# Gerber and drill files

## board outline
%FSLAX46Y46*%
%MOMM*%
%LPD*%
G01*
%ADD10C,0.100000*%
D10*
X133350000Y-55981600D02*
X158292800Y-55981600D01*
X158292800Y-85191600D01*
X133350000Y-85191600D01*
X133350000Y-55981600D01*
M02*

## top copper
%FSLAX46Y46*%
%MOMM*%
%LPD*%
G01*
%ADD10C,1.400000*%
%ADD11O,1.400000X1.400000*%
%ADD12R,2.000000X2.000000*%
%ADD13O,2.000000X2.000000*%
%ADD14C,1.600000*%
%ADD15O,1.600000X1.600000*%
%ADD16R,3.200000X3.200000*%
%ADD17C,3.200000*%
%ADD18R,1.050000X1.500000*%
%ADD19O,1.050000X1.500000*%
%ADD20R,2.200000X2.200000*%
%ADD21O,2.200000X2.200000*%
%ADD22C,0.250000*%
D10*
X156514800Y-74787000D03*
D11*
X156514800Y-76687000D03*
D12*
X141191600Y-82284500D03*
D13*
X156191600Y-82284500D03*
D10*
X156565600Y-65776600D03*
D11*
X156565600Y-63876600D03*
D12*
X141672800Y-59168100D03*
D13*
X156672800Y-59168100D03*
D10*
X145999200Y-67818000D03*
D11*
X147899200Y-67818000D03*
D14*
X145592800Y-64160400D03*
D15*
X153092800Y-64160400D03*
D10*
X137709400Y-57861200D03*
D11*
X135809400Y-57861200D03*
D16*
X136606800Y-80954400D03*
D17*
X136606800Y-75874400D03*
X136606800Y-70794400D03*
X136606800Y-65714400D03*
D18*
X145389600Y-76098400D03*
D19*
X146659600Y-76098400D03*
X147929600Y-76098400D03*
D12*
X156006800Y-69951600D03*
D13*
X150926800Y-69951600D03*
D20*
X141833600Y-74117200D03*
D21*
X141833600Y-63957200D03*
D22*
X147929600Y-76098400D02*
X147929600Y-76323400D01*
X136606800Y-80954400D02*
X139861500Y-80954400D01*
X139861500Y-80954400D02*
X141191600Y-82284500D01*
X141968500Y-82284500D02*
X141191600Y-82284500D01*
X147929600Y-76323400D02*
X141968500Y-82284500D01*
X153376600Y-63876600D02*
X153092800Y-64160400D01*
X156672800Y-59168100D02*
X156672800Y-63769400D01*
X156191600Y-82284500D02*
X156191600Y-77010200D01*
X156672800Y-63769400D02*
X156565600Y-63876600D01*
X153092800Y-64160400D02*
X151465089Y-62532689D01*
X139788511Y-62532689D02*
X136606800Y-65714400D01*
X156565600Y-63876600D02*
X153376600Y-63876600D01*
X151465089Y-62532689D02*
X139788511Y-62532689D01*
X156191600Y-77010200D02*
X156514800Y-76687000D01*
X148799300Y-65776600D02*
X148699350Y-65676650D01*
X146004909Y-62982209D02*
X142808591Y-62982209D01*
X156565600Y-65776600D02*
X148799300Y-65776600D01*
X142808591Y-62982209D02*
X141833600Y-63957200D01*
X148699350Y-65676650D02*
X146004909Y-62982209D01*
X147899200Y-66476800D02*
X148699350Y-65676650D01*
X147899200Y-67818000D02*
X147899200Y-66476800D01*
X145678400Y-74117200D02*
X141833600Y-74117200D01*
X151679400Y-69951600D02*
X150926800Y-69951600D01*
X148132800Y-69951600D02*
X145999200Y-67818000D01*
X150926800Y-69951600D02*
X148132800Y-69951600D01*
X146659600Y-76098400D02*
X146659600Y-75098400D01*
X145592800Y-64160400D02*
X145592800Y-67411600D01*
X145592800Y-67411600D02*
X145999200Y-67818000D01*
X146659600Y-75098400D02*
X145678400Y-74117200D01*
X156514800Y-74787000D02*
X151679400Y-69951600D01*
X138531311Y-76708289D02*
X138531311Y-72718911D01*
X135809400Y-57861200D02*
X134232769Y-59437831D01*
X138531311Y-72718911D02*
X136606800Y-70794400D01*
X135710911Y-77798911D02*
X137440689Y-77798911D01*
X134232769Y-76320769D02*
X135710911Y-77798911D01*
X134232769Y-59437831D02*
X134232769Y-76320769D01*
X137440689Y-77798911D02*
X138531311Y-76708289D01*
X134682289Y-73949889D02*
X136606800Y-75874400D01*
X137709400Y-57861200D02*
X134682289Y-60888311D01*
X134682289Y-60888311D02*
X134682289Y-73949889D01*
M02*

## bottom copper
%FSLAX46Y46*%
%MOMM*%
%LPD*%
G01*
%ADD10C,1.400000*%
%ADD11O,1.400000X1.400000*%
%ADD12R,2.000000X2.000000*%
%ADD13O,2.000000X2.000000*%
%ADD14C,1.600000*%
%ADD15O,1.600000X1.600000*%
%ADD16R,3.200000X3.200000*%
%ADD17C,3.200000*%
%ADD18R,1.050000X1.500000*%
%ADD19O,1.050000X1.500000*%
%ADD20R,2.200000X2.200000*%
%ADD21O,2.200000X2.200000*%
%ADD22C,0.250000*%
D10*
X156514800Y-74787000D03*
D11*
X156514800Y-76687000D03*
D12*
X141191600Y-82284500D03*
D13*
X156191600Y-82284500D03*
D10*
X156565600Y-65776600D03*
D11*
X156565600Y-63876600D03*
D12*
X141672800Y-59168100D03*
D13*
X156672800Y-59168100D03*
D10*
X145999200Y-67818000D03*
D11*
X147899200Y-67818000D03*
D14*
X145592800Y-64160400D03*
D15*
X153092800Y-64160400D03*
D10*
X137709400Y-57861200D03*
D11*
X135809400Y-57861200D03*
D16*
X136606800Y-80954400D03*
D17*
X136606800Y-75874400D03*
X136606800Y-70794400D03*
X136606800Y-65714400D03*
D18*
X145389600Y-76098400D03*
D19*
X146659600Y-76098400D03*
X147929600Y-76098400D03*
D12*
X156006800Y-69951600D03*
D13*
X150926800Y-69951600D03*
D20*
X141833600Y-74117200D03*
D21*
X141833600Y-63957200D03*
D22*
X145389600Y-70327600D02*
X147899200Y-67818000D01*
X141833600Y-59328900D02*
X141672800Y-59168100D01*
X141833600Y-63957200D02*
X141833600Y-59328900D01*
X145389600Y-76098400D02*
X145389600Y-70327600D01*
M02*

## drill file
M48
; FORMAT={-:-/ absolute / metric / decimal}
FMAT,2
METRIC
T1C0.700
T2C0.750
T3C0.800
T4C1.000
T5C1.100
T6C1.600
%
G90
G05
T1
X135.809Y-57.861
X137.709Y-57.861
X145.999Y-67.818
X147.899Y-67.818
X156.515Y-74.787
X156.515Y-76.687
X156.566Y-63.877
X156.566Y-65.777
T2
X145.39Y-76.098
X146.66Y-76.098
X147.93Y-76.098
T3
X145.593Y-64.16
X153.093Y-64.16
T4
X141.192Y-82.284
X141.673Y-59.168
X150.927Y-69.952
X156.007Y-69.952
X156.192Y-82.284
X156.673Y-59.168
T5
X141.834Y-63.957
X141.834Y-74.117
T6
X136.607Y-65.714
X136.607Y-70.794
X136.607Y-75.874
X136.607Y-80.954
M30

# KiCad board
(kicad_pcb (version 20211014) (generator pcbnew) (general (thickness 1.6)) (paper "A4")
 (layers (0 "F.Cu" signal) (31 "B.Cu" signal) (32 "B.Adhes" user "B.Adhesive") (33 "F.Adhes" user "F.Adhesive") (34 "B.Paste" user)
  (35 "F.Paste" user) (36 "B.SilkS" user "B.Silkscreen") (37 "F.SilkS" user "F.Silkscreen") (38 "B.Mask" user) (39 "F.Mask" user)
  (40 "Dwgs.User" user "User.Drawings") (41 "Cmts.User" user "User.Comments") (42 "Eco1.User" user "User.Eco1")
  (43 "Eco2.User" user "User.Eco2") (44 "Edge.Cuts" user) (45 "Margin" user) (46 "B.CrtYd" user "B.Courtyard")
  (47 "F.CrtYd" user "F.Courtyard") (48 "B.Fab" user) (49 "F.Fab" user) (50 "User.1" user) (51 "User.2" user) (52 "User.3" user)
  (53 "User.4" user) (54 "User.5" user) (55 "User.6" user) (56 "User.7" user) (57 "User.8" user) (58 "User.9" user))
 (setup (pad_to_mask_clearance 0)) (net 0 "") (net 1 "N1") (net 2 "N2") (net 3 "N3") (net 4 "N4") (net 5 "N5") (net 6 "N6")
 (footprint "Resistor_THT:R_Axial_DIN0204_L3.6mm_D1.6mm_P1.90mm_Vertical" (layer "F.Cu") (at 156.5148 74.787 -90)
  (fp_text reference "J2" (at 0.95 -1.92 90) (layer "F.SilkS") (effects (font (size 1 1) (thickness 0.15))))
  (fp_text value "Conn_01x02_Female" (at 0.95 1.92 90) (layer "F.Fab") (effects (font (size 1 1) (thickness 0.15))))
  (pad "1" thru_hole circle locked (at 0 0 270) (size 1.4 1.4) (drill 0.7) (layers *.Cu *.Mask) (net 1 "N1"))
  (pad "2" thru_hole oval locked (at 1.9 0 270) (size 1.4 1.4) (drill 0.7) (layers *.Cu *.Mask) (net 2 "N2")))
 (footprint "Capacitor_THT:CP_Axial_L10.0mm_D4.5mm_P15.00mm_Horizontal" (layer "F.Cu") (at 141.1916 82.2845)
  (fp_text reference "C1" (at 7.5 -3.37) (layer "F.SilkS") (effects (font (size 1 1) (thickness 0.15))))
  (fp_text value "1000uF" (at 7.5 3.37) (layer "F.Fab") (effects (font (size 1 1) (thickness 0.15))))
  (pad "1" thru_hole rect locked (at 0 0) (size 2 2) (drill 1) (layers *.Cu *.Mask) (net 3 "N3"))
  (pad "2" thru_hole oval locked (at 15 0) (size 2 2) (drill 1) (layers *.Cu *.Mask) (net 2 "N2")))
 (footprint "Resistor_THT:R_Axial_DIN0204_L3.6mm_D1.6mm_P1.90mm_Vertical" (layer "F.Cu") (at 156.5656 65.7766 90)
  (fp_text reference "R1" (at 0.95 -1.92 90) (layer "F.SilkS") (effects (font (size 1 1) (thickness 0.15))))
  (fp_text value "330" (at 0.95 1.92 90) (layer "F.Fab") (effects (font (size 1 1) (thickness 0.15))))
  (pad "1" thru_hole circle locked (at 0 0 90) (size 1.4 1.4) (drill 0.7) (layers *.Cu *.Mask) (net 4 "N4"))
  (pad "2" thru_hole oval locked (at 1.9 0 90) (size 1.4 1.4) (drill 0.7) (layers *.Cu *.Mask) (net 2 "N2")))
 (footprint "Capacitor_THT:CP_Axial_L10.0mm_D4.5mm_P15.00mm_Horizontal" (layer "F.Cu") (at 141.6728 59.1681)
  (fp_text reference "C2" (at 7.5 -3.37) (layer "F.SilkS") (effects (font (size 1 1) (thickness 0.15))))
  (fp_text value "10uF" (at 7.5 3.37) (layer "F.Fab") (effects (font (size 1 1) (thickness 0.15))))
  (pad "1" thru_hole rect locked (at 0 0) (size 2 2) (drill 1) (layers *.Cu *.Mask) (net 4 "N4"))
  (pad "2" thru_hole oval locked (at 15 0) (size 2 2) (drill 1) (layers *.Cu *.Mask) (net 2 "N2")))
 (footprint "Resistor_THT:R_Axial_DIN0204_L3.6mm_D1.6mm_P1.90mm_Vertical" (layer "F.Cu") (at 145.9992 67.818)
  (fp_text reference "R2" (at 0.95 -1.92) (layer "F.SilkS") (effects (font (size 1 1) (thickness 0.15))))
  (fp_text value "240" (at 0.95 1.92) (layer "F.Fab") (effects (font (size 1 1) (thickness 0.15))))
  (pad "1" thru_hole circle locked (at 0 0) (size 1.4 1.4) (drill 0.7) (layers *.Cu *.Mask) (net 1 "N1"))
  (pad "2" thru_hole oval locked (at 1.9 0) (size 1.4 1.4) (drill 0.7) (layers *.Cu *.Mask) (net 4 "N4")))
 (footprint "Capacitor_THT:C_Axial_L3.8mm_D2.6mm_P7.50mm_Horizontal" (layer "F.Cu") (at 145.5928 64.1604)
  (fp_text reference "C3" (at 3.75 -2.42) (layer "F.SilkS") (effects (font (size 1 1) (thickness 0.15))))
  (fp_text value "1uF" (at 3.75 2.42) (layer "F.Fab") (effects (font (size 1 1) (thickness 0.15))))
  (pad "1" thru_hole circle locked (at 0 0) (size 1.6 1.6) (drill 0.8) (layers *.Cu *.Mask) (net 1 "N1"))
  (pad "2" thru_hole oval locked (at 7.5 0) (size 1.6 1.6) (drill 0.8) (layers *.Cu *.Mask) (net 2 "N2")))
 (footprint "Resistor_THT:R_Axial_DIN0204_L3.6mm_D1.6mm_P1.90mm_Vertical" (layer "F.Cu") (at 137.7094 57.8612 180)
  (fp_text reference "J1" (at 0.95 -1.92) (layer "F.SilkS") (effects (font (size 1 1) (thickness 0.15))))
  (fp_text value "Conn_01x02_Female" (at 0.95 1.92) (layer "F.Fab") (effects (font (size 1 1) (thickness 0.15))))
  (pad "1" thru_hole circle locked (at 0 0 180) (size 1.4 1.4) (drill 0.7) (layers *.Cu *.Mask) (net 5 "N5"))
  (pad "2" thru_hole oval locked (at 1.9 0 180) (size 1.4 1.4) (drill 0.7) (layers *.Cu *.Mask) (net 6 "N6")))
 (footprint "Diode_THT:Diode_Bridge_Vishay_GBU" (layer "F.Cu") (at 136.6068 80.9544 90)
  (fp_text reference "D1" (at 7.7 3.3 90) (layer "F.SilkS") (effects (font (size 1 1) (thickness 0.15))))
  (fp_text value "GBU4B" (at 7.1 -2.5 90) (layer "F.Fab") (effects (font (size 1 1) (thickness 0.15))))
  (pad "1" thru_hole rect locked (at 0 0 90) (size 3.2 3.2) (drill 1.6) (layers *.Cu *.Mask) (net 3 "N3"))
  (pad "2" thru_hole circle locked (at 5.08 0 90) (size 3.2 3.2) (drill 1.6) (layers *.Cu *.Mask) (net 5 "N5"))
  (pad "3" thru_hole circle locked (at 10.16 0 90) (size 3.2 3.2) (drill 1.6) (layers *.Cu *.Mask) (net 6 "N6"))
  (pad "4" thru_hole circle locked (at 15.24 0 90) (size 3.2 3.2) (drill 1.6) (layers *.Cu *.Mask) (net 2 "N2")))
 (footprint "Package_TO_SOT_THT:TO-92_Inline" (layer "F.Cu") (at 145.3896 76.0984)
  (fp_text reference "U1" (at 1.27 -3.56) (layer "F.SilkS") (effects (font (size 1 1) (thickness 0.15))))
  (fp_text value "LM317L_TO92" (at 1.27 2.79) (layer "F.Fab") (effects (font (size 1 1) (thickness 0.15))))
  (pad "1" thru_hole rect locked (at 0 0) (size 1.05 1.5) (drill 0.75) (layers *.Cu *.Mask) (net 4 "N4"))
  (pad "2" thru_hole oval locked (at 1.27 0) (size 1.05 1.5) (drill 0.75) (layers *.Cu *.Mask) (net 1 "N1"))
  (pad "3" thru_hole oval locked (at 2.54 0) (size 1.05 1.5) (drill 0.75) (layers *.Cu *.Mask) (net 3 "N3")))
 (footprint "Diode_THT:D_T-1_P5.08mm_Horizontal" (layer "F.Cu") (at 156.0068 69.9516 180)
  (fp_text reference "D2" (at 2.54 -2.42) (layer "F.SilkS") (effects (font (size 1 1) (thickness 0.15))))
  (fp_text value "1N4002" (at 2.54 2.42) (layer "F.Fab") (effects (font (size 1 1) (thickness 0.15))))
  (pad "1" thru_hole rect locked (at 0 0 180) (size 2 2) (drill 1) (layers *.Cu *.Mask) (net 3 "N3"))
  (pad "2" thru_hole oval locked (at 5.08 0 180) (size 2 2) (drill 1) (layers *.Cu *.Mask) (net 1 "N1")))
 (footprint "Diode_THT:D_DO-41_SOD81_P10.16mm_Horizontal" (layer "F.Cu") (at 141.8336 74.1172 90)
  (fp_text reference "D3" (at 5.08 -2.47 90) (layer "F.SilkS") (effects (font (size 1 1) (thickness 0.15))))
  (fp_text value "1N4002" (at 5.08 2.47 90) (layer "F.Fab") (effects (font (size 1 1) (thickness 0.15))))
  (pad "1" thru_hole rect locked (at 0 0 90) (size 2.2 2.2) (drill 1.1) (layers *.Cu *.Mask) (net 1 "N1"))
  (pad "2" thru_hole oval locked (at 10.16 0 90) (size 2.2 2.2) (drill 1.1) (layers *.Cu *.Mask) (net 4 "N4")))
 (gr_rect (start 158.2928 55.9816) (end 133.35 85.1916) (layer "Edge.Cuts") (width 0.1) (fill none))
 (segment (start 147.9296 76.0984) (end 147.9296 76.3234) (width 0.25) (layer "F.Cu") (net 3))
 (segment (start 136.6068 80.9544) (end 139.8615 80.9544) (width 0.25) (layer "F.Cu") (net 3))
 (segment (start 139.8615 80.9544) (end 141.1916 82.2845) (width 0.25) (layer "F.Cu") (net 3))
 (segment (start 141.9685 82.2845) (end 141.1916 82.2845) (width 0.25) (layer "F.Cu") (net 3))
 (segment (start 147.9296 76.3234) (end 141.9685 82.2845) (width 0.25) (layer "F.Cu") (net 3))
 (segment (start 153.3766 63.8766) (end 153.0928 64.1604) (width 0.25) (layer "F.Cu") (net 2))
 (segment (start 156.6728 59.1681) (end 156.6728 63.7694) (width 0.25) (layer "F.Cu") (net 2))
 (segment (start 156.1916 82.2845) (end 156.1916 77.0102) (width 0.25) (layer "F.Cu") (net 2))
 (segment (start 156.6728 63.7694) (end 156.5656 63.8766) (width 0.25) (layer "F.Cu") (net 2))
 (segment (start 153.0928 64.1604) (end 151.465089 62.532689) (width 0.25) (layer "F.Cu") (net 2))
 (segment (start 139.788511 62.532689) (end 136.6068 65.7144) (width 0.25) (layer "F.Cu") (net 2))
 (segment (start 156.5656 63.8766) (end 153.3766 63.8766) (width 0.25) (layer "F.Cu") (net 2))
 (segment (start 151.465089 62.532689) (end 139.788511 62.532689) (width 0.25) (layer "F.Cu") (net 2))
 (segment (start 156.1916 77.0102) (end 156.5148 76.687) (width 0.25) (layer "F.Cu") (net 2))
 (segment (start 148.7993 65.7766) (end 148.69935 65.67665) (width 0.25) (layer "F.Cu") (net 4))
 (segment (start 146.004909 62.982209) (end 142.808591 62.982209) (width 0.25) (layer "F.Cu") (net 4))
 (segment (start 156.5656 65.7766) (end 148.7993 65.7766) (width 0.25) (layer "F.Cu") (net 4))
 (segment (start 142.808591 62.982209) (end 141.8336 63.9572) (width 0.25) (layer "F.Cu") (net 4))
 (segment (start 148.69935 65.67665) (end 146.004909 62.982209) (width 0.25) (layer "F.Cu") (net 4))
 (segment (start 147.8992 66.4768) (end 148.69935 65.67665) (width 0.25) (layer "F.Cu") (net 4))
 (segment (start 147.8992 67.818) (end 147.8992 66.4768) (width 0.25) (layer "F.Cu") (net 4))
 (segment (start 145.3896 70.3276) (end 147.8992 67.818) (width 0.25) (layer "B.Cu") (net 4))
 (segment (start 141.8336 59.3289) (end 141.6728 59.1681) (width 0.25) (layer "B.Cu") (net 4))
 (segment (start 141.8336 63.9572) (end 141.8336 59.3289) (width 0.25) (layer "B.Cu") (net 4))
 (segment (start 145.3896 76.0984) (end 145.3896 70.3276) (width 0.25) (layer "B.Cu") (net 4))
 (segment (start 145.6784 74.1172) (end 141.8336 74.1172) (width 0.25) (layer "F.Cu") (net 1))
 (segment (start 151.6794 69.9516) (end 150.9268 69.9516) (width 0.25) (layer "F.Cu") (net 1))
 (segment (start 148.1328 69.9516) (end 145.9992 67.818) (width 0.25) (layer "F.Cu") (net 1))
 (segment (start 150.9268 69.9516) (end 148.1328 69.9516) (width 0.25) (layer "F.Cu") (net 1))
 (segment (start 146.6596 76.0984) (end 146.6596 75.0984) (width 0.25) (layer "F.Cu") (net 1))
 (segment (start 145.5928 64.1604) (end 145.5928 67.4116) (width 0.25) (layer "F.Cu") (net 1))
 (segment (start 145.5928 67.4116) (end 145.9992 67.818) (width 0.25) (layer "F.Cu") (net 1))
 (segment (start 146.6596 75.0984) (end 145.6784 74.1172) (width 0.25) (layer "F.Cu") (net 1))
 (segment (start 156.5148 74.787) (end 151.6794 69.9516) (width 0.25) (layer "F.Cu") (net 1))
 (segment (start 138.531311 76.708289) (end 138.531311 72.718911) (width 0.25) (layer "F.Cu") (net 6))
 (segment (start 135.8094 57.8612) (end 134.232769 59.437831) (width 0.25) (layer "F.Cu") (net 6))
 (segment (start 138.531311 72.718911) (end 136.6068 70.7944) (width 0.25) (layer "F.Cu") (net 6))
 (segment (start 135.710911 77.798911) (end 137.440689 77.798911) (width 0.25) (layer "F.Cu") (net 6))
 (segment (start 134.232769 76.320769) (end 135.710911 77.798911) (width 0.25) (layer "F.Cu") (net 6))
 (segment (start 134.232769 59.437831) (end 134.232769 76.320769) (width 0.25) (layer "F.Cu") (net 6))
 (segment (start 137.440689 77.798911) (end 138.531311 76.708289) (width 0.25) (layer "F.Cu") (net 6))
 (segment (start 134.682289 73.949889) (end 136.6068 75.8744) (width 0.25) (layer "F.Cu") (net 5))
 (segment (start 137.7094 57.8612) (end 134.682289 60.888311) (width 0.25) (layer "F.Cu") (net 5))
 (segment (start 134.682289 60.888311) (end 134.682289 73.949889) (width 0.25) (layer "F.Cu") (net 5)))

